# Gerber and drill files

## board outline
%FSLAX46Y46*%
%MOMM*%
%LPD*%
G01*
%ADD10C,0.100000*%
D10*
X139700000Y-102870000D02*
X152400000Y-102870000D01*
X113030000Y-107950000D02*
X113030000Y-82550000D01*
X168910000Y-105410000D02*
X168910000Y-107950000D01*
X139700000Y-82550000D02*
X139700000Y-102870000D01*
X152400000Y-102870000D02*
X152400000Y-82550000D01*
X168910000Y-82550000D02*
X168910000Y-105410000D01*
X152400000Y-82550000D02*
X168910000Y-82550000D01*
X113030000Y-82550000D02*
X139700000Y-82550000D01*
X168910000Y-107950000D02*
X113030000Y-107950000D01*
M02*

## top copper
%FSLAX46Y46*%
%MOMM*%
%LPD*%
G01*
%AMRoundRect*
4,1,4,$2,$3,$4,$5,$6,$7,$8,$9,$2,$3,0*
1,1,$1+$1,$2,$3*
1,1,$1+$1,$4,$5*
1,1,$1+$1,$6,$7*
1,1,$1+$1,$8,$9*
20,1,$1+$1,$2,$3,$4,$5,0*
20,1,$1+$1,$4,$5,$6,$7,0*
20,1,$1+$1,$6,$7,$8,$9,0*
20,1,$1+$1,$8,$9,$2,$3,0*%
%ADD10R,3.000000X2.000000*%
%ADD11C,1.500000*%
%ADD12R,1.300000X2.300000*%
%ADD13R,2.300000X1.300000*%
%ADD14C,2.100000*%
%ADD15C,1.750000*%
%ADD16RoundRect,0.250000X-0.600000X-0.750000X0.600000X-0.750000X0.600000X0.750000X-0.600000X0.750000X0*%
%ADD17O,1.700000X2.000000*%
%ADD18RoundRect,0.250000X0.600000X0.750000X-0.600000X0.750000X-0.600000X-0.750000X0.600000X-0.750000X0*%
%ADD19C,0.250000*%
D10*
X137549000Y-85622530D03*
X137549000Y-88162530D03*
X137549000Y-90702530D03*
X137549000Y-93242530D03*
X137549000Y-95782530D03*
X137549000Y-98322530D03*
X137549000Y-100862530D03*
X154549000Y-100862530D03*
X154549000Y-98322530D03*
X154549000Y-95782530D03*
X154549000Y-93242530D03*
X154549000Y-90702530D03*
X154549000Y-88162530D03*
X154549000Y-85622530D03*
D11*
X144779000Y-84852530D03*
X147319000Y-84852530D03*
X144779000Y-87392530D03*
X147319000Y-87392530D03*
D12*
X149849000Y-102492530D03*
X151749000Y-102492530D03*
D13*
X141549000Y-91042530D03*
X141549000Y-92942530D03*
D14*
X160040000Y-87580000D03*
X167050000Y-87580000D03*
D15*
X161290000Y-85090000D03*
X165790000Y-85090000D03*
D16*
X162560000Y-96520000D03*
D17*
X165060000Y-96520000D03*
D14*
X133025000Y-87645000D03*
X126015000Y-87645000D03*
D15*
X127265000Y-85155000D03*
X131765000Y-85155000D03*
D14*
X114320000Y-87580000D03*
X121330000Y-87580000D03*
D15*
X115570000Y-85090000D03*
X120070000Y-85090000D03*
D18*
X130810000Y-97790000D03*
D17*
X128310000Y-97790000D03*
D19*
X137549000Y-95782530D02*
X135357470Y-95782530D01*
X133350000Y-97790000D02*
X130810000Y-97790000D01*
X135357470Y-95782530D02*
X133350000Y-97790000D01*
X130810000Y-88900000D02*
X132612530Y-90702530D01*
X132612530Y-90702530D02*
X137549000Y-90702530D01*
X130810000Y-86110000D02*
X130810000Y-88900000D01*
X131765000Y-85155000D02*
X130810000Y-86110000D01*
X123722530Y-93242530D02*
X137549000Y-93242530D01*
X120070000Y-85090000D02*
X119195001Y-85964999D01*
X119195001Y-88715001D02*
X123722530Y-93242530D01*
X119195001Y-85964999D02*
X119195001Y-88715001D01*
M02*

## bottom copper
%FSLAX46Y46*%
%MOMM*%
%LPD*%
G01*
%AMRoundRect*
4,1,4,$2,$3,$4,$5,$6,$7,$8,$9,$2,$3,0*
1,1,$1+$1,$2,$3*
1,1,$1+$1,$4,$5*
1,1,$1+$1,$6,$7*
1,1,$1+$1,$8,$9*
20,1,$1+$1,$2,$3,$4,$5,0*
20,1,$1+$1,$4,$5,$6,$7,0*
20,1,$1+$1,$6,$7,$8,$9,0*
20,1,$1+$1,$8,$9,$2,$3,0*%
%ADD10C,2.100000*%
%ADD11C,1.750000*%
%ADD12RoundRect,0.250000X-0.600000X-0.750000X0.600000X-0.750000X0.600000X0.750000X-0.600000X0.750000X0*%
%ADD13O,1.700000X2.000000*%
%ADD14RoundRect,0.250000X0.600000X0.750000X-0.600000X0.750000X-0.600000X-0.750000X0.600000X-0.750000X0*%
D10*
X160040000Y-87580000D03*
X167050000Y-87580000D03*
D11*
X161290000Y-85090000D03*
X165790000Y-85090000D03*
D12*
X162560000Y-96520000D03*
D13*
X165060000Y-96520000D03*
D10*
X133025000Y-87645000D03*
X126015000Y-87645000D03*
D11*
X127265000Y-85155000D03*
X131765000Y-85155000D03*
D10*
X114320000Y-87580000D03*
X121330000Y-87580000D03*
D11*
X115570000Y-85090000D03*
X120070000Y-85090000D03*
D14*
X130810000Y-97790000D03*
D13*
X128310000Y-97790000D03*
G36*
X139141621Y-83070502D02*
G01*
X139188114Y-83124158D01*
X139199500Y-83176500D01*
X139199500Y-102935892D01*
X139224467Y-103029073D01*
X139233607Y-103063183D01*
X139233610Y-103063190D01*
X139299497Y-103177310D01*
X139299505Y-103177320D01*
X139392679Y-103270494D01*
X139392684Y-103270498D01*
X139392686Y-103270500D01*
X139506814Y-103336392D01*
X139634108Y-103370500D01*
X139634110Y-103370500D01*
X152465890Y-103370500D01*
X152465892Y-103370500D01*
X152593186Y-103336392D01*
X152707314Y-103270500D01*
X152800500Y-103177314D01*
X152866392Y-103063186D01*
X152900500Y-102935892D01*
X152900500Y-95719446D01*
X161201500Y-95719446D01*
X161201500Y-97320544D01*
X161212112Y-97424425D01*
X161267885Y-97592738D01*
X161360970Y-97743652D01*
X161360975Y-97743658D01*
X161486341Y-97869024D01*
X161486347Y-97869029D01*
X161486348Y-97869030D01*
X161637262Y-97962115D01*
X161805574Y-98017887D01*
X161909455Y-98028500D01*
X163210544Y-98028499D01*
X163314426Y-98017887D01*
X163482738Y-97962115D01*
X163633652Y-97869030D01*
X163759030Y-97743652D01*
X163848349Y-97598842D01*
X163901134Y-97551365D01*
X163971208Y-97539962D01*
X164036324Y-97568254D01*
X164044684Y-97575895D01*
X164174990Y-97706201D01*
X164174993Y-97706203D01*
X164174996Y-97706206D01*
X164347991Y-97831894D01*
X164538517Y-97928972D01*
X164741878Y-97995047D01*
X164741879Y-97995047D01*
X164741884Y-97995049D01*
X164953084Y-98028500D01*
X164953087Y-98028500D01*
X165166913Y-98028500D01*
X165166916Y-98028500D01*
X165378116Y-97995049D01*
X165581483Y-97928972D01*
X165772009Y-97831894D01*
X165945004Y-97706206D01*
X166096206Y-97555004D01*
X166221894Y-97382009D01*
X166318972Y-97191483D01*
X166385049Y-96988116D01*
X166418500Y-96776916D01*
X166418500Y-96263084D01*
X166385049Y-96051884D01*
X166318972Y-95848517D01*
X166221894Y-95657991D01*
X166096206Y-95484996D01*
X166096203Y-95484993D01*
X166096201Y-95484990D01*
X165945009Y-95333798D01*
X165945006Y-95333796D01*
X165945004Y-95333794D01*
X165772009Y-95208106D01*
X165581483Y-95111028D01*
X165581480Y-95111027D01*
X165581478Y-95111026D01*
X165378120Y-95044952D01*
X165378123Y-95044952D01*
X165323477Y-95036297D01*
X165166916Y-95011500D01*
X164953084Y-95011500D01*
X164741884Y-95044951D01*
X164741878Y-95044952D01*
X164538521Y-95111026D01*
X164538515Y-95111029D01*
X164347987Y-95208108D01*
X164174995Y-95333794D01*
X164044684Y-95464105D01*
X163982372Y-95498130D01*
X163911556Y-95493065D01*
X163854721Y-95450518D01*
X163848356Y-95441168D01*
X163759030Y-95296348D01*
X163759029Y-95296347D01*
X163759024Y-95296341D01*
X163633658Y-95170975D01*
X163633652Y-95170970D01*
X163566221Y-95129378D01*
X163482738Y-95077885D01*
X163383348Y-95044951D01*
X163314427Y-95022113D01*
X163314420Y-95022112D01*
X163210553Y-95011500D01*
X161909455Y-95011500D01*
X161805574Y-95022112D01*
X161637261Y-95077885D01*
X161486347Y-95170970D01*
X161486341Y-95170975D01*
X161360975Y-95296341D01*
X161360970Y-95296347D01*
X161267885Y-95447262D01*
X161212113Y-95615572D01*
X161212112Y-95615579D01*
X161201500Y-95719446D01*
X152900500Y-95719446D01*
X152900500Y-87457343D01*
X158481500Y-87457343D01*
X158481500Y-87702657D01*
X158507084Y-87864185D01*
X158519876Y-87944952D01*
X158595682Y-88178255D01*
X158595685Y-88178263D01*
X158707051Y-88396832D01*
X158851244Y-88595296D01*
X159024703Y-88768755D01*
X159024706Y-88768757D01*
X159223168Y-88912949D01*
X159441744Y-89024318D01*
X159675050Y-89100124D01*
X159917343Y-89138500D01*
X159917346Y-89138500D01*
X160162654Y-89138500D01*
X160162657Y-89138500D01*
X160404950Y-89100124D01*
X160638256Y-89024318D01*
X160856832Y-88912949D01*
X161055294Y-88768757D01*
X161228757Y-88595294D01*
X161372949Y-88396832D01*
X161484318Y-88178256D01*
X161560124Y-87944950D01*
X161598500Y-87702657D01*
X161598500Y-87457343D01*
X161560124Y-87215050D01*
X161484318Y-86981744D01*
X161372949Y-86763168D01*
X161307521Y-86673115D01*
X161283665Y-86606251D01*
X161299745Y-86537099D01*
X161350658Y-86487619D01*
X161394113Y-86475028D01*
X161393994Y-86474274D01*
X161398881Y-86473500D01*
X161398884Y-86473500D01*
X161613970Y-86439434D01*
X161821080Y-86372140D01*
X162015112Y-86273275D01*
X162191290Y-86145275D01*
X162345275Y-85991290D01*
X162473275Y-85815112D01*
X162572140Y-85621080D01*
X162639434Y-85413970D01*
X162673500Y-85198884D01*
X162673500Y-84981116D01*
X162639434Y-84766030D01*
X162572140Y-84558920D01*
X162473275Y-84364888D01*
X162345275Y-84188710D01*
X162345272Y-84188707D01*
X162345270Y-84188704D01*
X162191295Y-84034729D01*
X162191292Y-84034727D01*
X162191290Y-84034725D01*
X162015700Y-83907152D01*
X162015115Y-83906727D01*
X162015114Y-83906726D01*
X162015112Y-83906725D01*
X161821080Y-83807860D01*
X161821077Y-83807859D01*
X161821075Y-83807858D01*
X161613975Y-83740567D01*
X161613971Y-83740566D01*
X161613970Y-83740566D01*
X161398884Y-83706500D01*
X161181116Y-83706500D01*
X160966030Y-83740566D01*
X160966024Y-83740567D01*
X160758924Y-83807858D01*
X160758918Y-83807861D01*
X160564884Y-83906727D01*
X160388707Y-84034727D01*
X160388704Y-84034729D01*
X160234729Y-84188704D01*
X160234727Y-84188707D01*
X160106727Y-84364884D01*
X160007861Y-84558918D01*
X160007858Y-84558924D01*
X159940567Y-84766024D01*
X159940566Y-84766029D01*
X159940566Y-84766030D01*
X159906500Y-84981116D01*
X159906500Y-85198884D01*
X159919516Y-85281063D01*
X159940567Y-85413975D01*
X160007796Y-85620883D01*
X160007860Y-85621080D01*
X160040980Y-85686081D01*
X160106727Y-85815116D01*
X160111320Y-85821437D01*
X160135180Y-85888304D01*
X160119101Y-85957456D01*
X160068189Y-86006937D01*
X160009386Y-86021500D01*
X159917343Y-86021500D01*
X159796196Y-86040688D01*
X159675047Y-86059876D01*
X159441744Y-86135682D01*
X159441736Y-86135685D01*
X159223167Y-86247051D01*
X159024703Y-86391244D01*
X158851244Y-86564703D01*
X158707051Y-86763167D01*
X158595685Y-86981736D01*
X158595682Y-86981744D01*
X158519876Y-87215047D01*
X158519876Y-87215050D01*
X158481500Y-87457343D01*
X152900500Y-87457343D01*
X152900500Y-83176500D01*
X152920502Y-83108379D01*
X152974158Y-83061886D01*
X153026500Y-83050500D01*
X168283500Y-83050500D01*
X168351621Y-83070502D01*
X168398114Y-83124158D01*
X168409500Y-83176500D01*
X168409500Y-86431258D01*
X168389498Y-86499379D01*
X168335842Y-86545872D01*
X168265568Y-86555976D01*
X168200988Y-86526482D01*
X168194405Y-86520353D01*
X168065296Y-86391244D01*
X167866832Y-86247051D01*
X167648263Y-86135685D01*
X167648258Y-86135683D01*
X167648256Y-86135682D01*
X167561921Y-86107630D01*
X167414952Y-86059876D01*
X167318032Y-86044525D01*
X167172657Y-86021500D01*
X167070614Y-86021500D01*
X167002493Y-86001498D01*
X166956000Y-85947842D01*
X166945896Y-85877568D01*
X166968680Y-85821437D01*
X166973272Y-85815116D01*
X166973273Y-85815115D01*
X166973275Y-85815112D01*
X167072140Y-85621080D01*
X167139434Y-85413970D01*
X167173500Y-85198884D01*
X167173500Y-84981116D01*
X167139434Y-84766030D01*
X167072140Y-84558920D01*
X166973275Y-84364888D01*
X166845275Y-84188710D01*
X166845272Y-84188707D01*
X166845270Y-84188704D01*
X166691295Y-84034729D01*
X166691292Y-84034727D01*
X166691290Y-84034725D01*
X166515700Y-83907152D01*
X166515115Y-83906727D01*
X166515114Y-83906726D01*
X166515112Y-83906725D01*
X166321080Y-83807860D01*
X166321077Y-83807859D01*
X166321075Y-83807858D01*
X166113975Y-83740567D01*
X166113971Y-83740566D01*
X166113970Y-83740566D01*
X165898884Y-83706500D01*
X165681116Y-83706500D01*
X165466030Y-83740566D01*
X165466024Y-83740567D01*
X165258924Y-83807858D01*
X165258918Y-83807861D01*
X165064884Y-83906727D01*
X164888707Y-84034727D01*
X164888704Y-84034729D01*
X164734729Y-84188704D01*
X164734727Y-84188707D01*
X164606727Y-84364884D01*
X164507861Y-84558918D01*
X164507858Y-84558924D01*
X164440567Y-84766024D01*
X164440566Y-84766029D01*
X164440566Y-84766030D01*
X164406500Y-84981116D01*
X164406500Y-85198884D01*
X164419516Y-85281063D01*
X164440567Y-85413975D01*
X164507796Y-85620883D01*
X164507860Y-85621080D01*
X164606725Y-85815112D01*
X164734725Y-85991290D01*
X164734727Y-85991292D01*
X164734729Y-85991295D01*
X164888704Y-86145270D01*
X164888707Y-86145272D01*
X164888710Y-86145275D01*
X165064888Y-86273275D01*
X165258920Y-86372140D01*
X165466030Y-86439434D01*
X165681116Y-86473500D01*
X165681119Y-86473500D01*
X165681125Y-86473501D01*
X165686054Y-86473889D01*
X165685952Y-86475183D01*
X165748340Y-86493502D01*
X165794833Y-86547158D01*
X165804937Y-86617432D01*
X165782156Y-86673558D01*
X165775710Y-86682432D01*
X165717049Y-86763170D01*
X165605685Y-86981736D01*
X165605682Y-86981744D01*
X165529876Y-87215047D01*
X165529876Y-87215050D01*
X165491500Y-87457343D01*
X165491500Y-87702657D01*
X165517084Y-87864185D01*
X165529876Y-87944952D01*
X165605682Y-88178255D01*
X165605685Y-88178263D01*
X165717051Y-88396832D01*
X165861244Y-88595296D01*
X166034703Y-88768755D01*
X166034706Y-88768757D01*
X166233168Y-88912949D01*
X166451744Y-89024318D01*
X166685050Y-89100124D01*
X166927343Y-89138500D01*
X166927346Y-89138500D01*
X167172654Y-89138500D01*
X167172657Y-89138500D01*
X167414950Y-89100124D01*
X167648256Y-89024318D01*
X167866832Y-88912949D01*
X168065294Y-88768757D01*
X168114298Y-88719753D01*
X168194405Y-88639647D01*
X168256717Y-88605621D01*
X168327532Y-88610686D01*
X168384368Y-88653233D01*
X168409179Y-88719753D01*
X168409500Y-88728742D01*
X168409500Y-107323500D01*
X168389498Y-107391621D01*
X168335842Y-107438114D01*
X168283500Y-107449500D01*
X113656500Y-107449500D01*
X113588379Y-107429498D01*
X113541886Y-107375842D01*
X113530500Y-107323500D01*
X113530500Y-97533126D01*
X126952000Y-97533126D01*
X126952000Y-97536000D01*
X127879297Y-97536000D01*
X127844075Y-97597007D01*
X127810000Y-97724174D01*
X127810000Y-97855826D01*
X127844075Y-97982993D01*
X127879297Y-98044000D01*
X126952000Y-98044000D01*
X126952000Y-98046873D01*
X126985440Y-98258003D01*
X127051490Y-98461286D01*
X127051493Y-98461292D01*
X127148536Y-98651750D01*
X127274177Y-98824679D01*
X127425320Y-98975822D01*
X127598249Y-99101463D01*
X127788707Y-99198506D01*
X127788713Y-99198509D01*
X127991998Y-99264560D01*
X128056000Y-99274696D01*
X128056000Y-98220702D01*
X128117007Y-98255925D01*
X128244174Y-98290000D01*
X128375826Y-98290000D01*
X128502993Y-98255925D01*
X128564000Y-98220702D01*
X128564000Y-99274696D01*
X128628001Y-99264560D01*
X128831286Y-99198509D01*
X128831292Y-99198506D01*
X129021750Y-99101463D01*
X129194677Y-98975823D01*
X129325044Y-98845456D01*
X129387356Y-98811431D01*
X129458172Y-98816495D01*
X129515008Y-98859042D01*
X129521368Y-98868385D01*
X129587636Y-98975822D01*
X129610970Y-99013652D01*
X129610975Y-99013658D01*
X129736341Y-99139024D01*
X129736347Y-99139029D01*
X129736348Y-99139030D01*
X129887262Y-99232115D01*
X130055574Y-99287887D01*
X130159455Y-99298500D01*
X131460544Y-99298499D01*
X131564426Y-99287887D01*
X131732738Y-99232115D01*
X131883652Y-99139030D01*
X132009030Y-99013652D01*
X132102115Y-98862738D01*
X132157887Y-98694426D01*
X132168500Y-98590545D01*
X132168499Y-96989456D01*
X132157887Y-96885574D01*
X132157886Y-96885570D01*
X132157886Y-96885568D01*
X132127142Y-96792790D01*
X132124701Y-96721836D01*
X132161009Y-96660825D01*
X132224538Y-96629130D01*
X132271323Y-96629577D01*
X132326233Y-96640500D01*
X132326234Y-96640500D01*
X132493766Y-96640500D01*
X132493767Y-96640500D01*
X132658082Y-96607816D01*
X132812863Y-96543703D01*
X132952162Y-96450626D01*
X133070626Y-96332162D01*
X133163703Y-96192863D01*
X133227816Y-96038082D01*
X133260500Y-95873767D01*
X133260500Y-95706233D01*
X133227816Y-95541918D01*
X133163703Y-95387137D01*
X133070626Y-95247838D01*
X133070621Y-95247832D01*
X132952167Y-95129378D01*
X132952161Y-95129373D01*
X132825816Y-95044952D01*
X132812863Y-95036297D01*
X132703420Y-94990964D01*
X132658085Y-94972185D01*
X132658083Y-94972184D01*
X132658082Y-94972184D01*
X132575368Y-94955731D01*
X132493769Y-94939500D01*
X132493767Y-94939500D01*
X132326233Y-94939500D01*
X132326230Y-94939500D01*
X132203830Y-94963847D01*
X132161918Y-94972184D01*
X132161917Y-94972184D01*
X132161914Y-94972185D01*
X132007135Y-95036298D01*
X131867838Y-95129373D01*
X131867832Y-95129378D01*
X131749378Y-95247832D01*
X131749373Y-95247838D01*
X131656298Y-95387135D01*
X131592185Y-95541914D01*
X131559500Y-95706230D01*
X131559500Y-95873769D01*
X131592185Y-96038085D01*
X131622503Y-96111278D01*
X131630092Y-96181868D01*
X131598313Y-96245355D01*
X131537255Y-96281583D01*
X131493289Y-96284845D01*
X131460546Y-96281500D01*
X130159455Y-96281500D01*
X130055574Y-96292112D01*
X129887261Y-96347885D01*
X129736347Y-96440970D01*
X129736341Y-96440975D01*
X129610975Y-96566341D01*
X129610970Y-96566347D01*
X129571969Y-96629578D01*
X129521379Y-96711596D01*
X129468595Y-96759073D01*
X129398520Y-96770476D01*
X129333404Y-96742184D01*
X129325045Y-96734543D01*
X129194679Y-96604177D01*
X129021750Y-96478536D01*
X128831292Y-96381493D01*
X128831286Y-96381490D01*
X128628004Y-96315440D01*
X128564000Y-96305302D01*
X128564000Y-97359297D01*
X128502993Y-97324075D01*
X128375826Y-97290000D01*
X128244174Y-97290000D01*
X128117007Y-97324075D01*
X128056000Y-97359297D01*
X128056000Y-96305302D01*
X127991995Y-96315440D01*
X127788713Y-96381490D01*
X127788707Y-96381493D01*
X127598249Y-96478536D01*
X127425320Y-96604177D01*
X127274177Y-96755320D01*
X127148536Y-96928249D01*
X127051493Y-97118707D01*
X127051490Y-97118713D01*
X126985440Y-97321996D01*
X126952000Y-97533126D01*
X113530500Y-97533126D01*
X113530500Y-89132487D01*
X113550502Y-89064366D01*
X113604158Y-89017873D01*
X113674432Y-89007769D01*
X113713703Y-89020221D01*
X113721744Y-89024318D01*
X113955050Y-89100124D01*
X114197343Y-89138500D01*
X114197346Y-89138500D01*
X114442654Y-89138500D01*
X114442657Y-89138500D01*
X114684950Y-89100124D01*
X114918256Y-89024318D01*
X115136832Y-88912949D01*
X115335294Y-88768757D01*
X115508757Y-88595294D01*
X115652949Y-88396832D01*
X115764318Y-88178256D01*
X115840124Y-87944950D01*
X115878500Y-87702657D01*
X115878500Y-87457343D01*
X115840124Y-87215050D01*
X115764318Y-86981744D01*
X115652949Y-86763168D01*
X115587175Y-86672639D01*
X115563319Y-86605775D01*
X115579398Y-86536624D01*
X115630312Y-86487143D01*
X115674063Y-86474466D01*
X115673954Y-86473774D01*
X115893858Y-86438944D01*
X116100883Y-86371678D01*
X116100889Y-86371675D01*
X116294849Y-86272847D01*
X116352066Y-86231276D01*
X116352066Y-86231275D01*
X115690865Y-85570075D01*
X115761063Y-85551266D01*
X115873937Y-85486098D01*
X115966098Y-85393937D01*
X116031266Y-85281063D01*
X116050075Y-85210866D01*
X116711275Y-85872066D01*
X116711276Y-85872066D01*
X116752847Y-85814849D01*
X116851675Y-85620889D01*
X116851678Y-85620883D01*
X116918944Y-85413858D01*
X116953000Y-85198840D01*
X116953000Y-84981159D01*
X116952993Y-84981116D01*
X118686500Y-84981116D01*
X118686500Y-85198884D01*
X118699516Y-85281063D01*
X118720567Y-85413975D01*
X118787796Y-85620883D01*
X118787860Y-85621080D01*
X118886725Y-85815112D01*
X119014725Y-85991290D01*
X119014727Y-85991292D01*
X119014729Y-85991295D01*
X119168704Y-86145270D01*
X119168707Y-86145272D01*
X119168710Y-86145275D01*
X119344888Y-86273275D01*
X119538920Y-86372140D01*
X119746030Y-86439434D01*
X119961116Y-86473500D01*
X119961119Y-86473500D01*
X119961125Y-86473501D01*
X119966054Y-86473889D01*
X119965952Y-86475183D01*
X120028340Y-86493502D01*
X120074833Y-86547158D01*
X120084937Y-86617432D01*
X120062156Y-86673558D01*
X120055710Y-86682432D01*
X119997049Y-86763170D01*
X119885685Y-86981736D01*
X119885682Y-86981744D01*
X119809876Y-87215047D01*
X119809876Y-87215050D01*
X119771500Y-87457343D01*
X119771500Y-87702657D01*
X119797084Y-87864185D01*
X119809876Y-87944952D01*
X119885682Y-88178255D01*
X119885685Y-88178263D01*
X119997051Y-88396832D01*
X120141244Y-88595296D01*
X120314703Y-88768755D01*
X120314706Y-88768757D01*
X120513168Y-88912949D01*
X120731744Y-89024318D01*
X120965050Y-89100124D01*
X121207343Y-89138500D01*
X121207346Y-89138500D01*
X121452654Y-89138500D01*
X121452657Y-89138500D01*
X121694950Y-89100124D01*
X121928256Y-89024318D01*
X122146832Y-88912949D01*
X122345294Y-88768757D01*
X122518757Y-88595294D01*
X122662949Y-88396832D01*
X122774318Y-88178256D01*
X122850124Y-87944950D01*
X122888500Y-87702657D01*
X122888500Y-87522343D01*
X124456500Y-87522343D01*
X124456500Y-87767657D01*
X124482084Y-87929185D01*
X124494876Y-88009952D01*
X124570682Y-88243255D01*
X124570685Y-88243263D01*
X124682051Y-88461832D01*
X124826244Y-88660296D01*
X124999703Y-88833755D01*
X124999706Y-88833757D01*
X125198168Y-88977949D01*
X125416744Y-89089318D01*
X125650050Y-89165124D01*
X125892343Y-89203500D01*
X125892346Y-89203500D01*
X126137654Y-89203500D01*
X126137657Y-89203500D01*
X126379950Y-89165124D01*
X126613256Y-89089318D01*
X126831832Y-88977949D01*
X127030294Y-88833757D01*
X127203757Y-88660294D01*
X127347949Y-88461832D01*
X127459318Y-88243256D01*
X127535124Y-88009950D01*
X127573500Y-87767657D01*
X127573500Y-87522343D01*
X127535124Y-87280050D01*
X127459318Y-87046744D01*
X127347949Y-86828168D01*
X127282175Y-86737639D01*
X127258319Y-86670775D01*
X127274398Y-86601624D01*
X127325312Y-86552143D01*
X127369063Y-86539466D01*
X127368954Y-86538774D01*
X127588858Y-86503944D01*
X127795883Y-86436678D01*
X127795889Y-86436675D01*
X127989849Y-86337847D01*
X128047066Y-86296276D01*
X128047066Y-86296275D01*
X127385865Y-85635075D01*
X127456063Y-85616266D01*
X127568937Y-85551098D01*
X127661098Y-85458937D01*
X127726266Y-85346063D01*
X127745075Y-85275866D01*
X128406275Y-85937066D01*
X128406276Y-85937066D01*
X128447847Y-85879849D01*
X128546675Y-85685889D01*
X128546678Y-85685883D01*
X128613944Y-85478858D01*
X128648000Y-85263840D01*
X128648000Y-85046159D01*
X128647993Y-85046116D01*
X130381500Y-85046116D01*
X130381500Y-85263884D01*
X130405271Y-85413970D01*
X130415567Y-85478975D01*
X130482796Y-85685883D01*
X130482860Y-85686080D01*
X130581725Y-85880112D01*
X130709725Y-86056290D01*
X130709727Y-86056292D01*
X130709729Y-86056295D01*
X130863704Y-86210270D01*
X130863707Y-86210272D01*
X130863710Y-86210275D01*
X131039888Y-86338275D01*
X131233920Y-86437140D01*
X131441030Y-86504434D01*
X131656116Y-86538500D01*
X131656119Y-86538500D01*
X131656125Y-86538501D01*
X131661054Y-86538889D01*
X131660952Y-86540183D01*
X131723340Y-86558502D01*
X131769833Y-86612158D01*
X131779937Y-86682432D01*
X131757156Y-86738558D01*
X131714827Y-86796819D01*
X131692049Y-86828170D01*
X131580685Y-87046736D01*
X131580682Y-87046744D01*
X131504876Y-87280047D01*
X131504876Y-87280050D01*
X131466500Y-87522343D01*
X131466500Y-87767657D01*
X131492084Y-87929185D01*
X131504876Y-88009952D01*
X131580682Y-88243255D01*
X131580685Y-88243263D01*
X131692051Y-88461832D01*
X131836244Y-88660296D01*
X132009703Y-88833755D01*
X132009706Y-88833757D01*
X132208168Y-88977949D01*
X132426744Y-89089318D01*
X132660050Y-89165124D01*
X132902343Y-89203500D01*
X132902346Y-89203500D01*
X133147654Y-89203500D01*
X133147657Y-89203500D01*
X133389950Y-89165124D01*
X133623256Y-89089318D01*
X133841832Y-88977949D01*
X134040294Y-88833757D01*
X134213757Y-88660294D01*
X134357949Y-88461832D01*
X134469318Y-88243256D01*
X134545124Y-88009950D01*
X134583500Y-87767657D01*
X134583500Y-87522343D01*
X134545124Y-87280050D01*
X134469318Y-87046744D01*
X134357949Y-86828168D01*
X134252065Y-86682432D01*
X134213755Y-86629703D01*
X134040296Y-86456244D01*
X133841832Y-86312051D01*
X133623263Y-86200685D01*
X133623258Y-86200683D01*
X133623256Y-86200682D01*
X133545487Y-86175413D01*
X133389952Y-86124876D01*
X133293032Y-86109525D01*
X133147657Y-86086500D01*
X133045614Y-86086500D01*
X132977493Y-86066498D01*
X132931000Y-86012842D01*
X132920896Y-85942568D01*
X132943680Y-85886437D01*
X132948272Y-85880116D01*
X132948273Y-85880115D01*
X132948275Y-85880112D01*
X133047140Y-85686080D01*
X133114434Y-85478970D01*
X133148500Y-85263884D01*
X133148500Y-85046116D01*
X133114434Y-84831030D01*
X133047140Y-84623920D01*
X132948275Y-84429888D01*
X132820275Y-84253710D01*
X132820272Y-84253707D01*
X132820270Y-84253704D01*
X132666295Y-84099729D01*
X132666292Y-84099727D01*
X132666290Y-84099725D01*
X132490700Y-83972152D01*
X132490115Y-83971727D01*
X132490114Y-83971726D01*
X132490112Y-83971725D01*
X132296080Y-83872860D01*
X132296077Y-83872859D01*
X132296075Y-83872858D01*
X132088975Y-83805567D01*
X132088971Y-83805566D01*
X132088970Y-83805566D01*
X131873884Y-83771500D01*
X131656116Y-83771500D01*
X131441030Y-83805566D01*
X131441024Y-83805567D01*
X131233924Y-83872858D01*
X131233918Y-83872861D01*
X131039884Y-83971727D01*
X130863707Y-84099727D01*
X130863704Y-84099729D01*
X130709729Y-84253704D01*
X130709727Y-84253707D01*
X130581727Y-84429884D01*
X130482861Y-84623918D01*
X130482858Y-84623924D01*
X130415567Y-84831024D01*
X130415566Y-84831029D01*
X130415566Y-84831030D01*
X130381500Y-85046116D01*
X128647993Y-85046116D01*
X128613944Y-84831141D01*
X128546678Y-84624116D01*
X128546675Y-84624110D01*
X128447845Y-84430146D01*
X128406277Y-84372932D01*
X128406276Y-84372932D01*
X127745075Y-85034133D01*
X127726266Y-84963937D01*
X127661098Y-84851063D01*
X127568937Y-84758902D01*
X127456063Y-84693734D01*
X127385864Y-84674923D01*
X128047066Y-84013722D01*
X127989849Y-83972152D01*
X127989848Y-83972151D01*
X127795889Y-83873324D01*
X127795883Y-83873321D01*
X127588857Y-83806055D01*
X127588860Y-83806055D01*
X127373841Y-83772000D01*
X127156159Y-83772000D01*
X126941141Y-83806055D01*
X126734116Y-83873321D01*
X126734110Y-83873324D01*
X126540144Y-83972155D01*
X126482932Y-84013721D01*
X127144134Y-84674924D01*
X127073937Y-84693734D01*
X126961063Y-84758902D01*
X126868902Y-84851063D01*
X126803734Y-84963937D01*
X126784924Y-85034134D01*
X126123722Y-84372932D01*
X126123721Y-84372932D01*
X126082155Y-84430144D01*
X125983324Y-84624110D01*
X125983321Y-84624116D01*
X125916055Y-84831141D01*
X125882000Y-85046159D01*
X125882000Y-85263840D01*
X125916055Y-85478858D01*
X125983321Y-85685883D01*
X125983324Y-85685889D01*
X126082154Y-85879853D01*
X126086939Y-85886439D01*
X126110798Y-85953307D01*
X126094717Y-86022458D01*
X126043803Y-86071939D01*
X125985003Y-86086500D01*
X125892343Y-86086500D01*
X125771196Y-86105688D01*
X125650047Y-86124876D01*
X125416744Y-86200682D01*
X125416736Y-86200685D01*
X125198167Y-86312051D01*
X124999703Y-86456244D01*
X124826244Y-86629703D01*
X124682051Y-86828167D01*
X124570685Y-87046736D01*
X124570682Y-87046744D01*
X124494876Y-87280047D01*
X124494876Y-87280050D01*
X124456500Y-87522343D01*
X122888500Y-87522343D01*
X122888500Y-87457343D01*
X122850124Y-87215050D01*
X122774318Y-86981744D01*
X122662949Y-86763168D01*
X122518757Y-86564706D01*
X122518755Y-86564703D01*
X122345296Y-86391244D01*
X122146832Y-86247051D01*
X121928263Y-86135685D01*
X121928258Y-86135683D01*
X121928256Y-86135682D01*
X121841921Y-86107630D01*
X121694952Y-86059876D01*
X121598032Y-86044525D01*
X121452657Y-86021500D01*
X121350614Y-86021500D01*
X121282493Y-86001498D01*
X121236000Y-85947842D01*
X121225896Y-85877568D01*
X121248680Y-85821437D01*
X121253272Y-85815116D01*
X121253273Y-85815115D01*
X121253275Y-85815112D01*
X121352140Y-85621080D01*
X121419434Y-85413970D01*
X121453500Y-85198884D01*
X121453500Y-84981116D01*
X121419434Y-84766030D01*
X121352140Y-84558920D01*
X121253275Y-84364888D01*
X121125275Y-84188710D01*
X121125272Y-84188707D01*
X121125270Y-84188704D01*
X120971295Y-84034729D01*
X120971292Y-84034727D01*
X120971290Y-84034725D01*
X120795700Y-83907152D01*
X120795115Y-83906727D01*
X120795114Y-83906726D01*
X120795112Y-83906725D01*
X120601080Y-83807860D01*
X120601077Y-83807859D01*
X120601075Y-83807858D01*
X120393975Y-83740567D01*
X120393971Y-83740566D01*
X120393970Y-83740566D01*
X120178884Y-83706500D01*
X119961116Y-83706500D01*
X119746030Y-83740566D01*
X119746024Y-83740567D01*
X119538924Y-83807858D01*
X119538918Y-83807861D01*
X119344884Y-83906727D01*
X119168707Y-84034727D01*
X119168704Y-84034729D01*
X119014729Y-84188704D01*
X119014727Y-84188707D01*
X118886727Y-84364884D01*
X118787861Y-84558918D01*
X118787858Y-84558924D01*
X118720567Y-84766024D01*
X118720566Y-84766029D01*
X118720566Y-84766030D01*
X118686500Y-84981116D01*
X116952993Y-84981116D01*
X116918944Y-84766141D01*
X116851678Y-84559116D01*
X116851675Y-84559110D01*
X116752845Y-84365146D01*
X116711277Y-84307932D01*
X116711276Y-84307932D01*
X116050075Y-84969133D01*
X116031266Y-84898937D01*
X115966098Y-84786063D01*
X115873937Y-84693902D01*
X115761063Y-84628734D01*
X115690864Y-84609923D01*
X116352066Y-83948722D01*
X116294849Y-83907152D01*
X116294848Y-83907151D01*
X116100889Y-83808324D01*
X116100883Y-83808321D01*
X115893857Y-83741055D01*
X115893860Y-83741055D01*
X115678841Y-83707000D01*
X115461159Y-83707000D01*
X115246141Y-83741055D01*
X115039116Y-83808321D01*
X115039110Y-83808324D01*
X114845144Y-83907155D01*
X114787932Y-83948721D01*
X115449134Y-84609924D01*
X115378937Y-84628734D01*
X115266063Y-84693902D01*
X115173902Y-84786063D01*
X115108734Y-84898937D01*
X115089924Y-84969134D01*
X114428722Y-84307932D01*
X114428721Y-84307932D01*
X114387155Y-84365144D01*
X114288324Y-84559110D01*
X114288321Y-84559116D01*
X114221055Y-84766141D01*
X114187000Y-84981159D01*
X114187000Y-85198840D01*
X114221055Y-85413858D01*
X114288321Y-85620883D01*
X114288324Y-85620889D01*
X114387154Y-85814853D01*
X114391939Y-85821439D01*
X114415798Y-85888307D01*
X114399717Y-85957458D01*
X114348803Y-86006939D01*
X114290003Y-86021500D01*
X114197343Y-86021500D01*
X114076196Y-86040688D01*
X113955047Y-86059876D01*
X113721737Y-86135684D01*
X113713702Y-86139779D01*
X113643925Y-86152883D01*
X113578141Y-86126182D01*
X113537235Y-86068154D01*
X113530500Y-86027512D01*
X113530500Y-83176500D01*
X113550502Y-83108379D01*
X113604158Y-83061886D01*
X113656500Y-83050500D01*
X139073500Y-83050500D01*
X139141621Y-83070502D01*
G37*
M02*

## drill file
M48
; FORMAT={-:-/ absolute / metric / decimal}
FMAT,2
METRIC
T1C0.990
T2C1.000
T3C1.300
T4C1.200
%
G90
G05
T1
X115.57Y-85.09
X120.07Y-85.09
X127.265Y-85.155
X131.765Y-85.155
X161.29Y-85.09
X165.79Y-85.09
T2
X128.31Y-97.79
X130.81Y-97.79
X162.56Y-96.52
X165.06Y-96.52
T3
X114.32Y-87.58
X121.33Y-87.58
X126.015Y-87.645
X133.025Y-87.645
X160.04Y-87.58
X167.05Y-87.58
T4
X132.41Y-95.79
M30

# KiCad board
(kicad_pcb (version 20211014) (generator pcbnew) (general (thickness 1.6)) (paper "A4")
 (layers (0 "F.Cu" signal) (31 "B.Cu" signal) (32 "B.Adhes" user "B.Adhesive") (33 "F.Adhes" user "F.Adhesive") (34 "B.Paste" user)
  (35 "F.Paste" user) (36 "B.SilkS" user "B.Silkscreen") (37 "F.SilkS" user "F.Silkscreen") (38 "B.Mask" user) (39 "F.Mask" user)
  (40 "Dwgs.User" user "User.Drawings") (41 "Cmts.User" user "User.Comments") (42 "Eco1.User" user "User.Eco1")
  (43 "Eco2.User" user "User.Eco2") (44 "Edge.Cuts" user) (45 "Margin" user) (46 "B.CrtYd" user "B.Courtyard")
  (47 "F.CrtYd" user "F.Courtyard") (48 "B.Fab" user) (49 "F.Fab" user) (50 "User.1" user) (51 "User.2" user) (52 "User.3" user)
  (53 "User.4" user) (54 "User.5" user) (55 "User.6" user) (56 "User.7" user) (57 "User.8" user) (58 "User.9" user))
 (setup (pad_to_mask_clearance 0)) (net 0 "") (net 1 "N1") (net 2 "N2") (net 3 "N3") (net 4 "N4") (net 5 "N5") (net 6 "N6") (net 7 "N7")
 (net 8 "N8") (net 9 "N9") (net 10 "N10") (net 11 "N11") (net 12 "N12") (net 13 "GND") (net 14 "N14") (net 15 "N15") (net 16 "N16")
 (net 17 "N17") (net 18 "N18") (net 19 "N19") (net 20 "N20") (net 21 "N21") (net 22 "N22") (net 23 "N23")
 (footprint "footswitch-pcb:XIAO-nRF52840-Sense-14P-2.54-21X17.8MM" (layer "F.Cu") (at 146.049 93.24253)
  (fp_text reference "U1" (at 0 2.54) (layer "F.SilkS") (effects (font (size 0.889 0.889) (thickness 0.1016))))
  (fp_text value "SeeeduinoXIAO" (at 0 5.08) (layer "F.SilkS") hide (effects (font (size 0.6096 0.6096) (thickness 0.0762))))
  (pad "1" smd rect (at -8.5 -7.62) (size 3 2) (layers "F.Cu" "F.Paste" "F.Mask") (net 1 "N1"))
  (pad "2" smd rect (at -8.5 -5.08) (size 3 2) (layers "F.Cu" "F.Paste" "F.Mask") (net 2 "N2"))
  (pad "3" smd rect (at -8.5 -2.54) (size 3 2) (layers "F.Cu" "F.Paste" "F.Mask") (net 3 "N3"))
  (pad "4" smd rect (at -8.5 0) (size 3 2) (layers "F.Cu" "F.Paste" "F.Mask") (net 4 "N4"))
  (pad "5" smd rect (at -8.5 2.54) (size 3 2) (layers "F.Cu" "F.Paste" "F.Mask") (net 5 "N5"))
  (pad "6" smd rect (at -8.5 5.08 180) (size 3 2) (layers "F.Cu" "F.Paste" "F.Mask") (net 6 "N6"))
  (pad "7" smd rect (at -8.5 7.62) (size 3 2) (layers "F.Cu" "F.Paste" "F.Mask") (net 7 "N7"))
  (pad "8" smd rect (at 8.5 7.62) (size 3 2) (layers "F.Cu" "F.Paste" "F.Mask") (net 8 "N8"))
  (pad "9" smd rect (at 8.5 5.08) (size 3 2) (layers "F.Cu" "F.Paste" "F.Mask") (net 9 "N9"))
  (pad "10" smd rect (at 8.5 2.54) (size 3 2) (layers "F.Cu" "F.Paste" "F.Mask") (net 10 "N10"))
  (pad "11" smd rect (at 8.5 0) (size 3 2) (layers "F.Cu" "F.Paste" "F.Mask") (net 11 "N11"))
  (pad "12" smd rect (at 8.5 -2.54) (size 3 2) (layers "F.Cu" "F.Paste" "F.Mask") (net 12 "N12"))
  (pad "13" smd rect (at 8.5 -5.08) (size 3 2) (layers "F.Cu" "F.Paste" "F.Mask") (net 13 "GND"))
  (pad "14" smd rect (at 8.5 -7.62) (size 3 2) (layers "F.Cu" "F.Paste" "F.Mask") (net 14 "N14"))
  (pad "15" smd circle (at -1.27 -8.39 90) (size 1.5 1.5) (layers "F.Cu" "F.Paste" "F.Mask") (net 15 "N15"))
  (pad "16" smd circle (at 1.27 -8.39 90) (size 1.5 1.5) (layers "F.Cu" "F.Paste" "F.Mask") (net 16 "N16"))
  (pad "17" smd circle (at -1.27 -5.85 90) (size 1.5 1.5) (layers "F.Cu" "F.Paste" "F.Mask") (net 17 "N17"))
  (pad "18" smd circle (at 1.27 -5.85 90) (size 1.5 1.5) (layers "F.Cu" "F.Paste" "F.Mask") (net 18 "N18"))
  (pad "19" smd rect (at 3.8 9.25 90) (size 2.3 1.3) (layers "F.Cu" "F.Paste" "F.Mask") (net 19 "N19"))
  (pad "20" smd rect (at 5.7 9.25 90) (size 2.3 1.3) (layers "F.Cu" "F.Paste" "F.Mask") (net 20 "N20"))
  (pad "21" smd rect (at -4.5 -2.2 180) (size 2.3 1.3) (layers "F.Cu" "F.Paste" "F.Mask") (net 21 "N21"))
  (pad "22" smd rect (at -4.5 -0.3 180) (size 2.3 1.3) (layers "F.Cu" "F.Paste" "F.Mask") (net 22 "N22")))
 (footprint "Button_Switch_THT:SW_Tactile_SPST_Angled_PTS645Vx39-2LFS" (layer "F.Cu") (at 161.29 85.09)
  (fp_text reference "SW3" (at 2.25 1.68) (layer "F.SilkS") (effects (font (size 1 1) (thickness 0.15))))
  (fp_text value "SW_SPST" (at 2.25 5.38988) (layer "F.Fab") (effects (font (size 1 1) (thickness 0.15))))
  (pad "" thru_hole circle (at -1.25 2.49) (size 2.1 2.1) (drill 1.3) (layers *.Cu *.Mask))
  (pad "" thru_hole circle (at 5.76 2.49) (size 2.1 2.1) (drill 1.3) (layers *.Cu *.Mask))
  (pad "1" thru_hole circle (at 0 0) (size 1.75 1.75) (drill 0.99) (layers *.Cu *.Mask) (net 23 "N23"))
  (pad "2" thru_hole circle (at 4.5 0) (size 1.75 1.75) (drill 0.99) (layers *.Cu *.Mask) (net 22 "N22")))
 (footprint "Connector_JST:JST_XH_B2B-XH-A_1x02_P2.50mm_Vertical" (layer "F.Cu") (at 162.56 96.52)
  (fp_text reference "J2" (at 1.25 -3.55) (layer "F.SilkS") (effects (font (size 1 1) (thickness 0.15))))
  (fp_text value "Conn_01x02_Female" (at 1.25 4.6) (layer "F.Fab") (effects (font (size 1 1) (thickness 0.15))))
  (pad "1" thru_hole roundrect (at 0 0) (size 1.7 2) (drill 1) (layers *.Cu *.Mask) (roundrect_rratio 0.147059) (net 21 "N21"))
  (pad "2" thru_hole oval (at 2.5 0) (size 1.7 2) (drill 1) (layers *.Cu *.Mask) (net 23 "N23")))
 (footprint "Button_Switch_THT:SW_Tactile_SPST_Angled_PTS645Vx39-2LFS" (layer "F.Cu") (at 127.265 85.155)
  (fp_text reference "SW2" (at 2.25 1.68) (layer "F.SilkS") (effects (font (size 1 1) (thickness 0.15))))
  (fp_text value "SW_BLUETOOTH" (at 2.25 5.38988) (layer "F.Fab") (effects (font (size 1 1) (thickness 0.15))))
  (pad "" thru_hole circle (at 5.76 2.49) (size 2.1 2.1) (drill 1.3) (layers *.Cu *.Mask))
  (pad "" thru_hole circle (at -1.25 2.49) (size 2.1 2.1) (drill 1.3) (layers *.Cu *.Mask))
  (pad "1" thru_hole circle (at 0 0) (size 1.75 1.75) (drill 0.99) (layers *.Cu *.Mask) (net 13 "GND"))
  (pad "2" thru_hole circle (at 4.5 0) (size 1.75 1.75) (drill 0.99) (layers *.Cu *.Mask) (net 3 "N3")))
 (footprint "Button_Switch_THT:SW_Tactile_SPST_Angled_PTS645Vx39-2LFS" (layer "F.Cu") (at 115.57 85.09)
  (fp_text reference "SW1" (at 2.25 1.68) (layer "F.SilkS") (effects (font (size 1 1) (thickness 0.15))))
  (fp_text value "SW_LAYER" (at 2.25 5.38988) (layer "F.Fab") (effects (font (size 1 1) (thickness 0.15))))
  (pad "" thru_hole circle (at -1.25 2.49) (size 2.1 2.1) (drill 1.3) (layers *.Cu *.Mask))
  (pad "" thru_hole circle (at 5.76 2.49) (size 2.1 2.1) (drill 1.3) (layers *.Cu *.Mask))
  (pad "1" thru_hole circle (at 0 0) (size 1.75 1.75) (drill 0.99) (layers *.Cu *.Mask) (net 13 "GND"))
  (pad "2" thru_hole circle (at 4.5 0) (size 1.75 1.75) (drill 0.99) (layers *.Cu *.Mask) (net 4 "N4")))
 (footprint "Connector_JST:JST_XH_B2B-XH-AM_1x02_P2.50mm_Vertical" (layer "F.Cu") (at 130.81 97.79 180)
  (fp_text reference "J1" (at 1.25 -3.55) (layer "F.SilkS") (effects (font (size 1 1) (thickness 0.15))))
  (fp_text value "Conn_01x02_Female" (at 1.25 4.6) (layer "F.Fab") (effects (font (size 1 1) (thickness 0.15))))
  (pad "" np_thru_hole circle (at -1.6 2 180) (size 1.2 1.2) (drill 1.2) (layers *.Cu *.Mask))
  (pad "1" thru_hole roundrect (at 0 0 180) (size 1.7 2) (drill 1) (layers *.Cu *.Mask) (roundrect_rratio 0.147059) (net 5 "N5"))
  (pad "2" thru_hole oval (at 2.5 0 180) (size 1.7 2) (drill 1) (layers *.Cu *.Mask) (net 13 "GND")))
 (gr_line (start 139.7 102.87) (end 152.4 102.87) (layer "Edge.Cuts") (width 0.1))
 (gr_line (start 113.03 107.95) (end 113.03 82.55) (layer "Edge.Cuts") (width 0.1))
 (gr_line (start 168.91 105.41) (end 168.91 107.95) (layer "Edge.Cuts") (width 0.1))
 (gr_line (start 139.7 82.55) (end 139.7 102.87) (layer "Edge.Cuts") (width 0.1))
 (gr_line (start 152.4 102.87) (end 152.4 82.55) (layer "Edge.Cuts") (width 0.1))
 (gr_line (start 168.91 82.55) (end 168.91 105.41) (layer "Edge.Cuts") (width 0.1))
 (gr_line (start 152.4 82.55) (end 168.91 82.55) (layer "Edge.Cuts") (width 0.1))
 (gr_line (start 113.03 82.55) (end 139.7 82.55) (layer "Edge.Cuts") (width 0.1))
 (gr_line (start 168.91 107.95) (end 113.03 107.95) (layer "Edge.Cuts") (width 0.1))
 (segment (start 137.549 95.78253) (end 135.35747 95.78253) (width 0.25) (layer "F.Cu") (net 5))
 (segment (start 133.35 97.79) (end 130.81 97.79) (width 0.25) (layer "F.Cu") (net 5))
 (segment (start 135.35747 95.78253) (end 133.35 97.79) (width 0.25) (layer "F.Cu") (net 5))
 (segment (start 130.81 88.9) (end 132.61253 90.70253) (width 0.25) (layer "F.Cu") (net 3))
 (segment (start 132.61253 90.70253) (end 137.549 90.70253) (width 0.25) (layer "F.Cu") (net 3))
 (segment (start 130.81 86.11) (end 130.81 88.9) (width 0.25) (layer "F.Cu") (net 3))
 (segment (start 131.765 85.155) (end 130.81 86.11) (width 0.25) (layer "F.Cu") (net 3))
 (segment (start 123.72253 93.24253) (end 137.549 93.24253) (width 0.25) (layer "F.Cu") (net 4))
 (segment (start 120.07 85.09) (end 119.195001 85.964999) (width 0.25) (layer "F.Cu") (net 4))
 (segment (start 119.195001 88.715001) (end 123.72253 93.24253) (width 0.25) (layer "F.Cu") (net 4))
 (segment (start 119.195001 85.964999) (end 119.195001 88.715001) (width 0.25) (layer "F.Cu") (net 4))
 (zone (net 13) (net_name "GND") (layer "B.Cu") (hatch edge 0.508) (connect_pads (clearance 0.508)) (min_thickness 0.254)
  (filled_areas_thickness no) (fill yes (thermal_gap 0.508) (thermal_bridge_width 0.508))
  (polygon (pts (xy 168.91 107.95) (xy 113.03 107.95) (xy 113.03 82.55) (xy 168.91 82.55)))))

